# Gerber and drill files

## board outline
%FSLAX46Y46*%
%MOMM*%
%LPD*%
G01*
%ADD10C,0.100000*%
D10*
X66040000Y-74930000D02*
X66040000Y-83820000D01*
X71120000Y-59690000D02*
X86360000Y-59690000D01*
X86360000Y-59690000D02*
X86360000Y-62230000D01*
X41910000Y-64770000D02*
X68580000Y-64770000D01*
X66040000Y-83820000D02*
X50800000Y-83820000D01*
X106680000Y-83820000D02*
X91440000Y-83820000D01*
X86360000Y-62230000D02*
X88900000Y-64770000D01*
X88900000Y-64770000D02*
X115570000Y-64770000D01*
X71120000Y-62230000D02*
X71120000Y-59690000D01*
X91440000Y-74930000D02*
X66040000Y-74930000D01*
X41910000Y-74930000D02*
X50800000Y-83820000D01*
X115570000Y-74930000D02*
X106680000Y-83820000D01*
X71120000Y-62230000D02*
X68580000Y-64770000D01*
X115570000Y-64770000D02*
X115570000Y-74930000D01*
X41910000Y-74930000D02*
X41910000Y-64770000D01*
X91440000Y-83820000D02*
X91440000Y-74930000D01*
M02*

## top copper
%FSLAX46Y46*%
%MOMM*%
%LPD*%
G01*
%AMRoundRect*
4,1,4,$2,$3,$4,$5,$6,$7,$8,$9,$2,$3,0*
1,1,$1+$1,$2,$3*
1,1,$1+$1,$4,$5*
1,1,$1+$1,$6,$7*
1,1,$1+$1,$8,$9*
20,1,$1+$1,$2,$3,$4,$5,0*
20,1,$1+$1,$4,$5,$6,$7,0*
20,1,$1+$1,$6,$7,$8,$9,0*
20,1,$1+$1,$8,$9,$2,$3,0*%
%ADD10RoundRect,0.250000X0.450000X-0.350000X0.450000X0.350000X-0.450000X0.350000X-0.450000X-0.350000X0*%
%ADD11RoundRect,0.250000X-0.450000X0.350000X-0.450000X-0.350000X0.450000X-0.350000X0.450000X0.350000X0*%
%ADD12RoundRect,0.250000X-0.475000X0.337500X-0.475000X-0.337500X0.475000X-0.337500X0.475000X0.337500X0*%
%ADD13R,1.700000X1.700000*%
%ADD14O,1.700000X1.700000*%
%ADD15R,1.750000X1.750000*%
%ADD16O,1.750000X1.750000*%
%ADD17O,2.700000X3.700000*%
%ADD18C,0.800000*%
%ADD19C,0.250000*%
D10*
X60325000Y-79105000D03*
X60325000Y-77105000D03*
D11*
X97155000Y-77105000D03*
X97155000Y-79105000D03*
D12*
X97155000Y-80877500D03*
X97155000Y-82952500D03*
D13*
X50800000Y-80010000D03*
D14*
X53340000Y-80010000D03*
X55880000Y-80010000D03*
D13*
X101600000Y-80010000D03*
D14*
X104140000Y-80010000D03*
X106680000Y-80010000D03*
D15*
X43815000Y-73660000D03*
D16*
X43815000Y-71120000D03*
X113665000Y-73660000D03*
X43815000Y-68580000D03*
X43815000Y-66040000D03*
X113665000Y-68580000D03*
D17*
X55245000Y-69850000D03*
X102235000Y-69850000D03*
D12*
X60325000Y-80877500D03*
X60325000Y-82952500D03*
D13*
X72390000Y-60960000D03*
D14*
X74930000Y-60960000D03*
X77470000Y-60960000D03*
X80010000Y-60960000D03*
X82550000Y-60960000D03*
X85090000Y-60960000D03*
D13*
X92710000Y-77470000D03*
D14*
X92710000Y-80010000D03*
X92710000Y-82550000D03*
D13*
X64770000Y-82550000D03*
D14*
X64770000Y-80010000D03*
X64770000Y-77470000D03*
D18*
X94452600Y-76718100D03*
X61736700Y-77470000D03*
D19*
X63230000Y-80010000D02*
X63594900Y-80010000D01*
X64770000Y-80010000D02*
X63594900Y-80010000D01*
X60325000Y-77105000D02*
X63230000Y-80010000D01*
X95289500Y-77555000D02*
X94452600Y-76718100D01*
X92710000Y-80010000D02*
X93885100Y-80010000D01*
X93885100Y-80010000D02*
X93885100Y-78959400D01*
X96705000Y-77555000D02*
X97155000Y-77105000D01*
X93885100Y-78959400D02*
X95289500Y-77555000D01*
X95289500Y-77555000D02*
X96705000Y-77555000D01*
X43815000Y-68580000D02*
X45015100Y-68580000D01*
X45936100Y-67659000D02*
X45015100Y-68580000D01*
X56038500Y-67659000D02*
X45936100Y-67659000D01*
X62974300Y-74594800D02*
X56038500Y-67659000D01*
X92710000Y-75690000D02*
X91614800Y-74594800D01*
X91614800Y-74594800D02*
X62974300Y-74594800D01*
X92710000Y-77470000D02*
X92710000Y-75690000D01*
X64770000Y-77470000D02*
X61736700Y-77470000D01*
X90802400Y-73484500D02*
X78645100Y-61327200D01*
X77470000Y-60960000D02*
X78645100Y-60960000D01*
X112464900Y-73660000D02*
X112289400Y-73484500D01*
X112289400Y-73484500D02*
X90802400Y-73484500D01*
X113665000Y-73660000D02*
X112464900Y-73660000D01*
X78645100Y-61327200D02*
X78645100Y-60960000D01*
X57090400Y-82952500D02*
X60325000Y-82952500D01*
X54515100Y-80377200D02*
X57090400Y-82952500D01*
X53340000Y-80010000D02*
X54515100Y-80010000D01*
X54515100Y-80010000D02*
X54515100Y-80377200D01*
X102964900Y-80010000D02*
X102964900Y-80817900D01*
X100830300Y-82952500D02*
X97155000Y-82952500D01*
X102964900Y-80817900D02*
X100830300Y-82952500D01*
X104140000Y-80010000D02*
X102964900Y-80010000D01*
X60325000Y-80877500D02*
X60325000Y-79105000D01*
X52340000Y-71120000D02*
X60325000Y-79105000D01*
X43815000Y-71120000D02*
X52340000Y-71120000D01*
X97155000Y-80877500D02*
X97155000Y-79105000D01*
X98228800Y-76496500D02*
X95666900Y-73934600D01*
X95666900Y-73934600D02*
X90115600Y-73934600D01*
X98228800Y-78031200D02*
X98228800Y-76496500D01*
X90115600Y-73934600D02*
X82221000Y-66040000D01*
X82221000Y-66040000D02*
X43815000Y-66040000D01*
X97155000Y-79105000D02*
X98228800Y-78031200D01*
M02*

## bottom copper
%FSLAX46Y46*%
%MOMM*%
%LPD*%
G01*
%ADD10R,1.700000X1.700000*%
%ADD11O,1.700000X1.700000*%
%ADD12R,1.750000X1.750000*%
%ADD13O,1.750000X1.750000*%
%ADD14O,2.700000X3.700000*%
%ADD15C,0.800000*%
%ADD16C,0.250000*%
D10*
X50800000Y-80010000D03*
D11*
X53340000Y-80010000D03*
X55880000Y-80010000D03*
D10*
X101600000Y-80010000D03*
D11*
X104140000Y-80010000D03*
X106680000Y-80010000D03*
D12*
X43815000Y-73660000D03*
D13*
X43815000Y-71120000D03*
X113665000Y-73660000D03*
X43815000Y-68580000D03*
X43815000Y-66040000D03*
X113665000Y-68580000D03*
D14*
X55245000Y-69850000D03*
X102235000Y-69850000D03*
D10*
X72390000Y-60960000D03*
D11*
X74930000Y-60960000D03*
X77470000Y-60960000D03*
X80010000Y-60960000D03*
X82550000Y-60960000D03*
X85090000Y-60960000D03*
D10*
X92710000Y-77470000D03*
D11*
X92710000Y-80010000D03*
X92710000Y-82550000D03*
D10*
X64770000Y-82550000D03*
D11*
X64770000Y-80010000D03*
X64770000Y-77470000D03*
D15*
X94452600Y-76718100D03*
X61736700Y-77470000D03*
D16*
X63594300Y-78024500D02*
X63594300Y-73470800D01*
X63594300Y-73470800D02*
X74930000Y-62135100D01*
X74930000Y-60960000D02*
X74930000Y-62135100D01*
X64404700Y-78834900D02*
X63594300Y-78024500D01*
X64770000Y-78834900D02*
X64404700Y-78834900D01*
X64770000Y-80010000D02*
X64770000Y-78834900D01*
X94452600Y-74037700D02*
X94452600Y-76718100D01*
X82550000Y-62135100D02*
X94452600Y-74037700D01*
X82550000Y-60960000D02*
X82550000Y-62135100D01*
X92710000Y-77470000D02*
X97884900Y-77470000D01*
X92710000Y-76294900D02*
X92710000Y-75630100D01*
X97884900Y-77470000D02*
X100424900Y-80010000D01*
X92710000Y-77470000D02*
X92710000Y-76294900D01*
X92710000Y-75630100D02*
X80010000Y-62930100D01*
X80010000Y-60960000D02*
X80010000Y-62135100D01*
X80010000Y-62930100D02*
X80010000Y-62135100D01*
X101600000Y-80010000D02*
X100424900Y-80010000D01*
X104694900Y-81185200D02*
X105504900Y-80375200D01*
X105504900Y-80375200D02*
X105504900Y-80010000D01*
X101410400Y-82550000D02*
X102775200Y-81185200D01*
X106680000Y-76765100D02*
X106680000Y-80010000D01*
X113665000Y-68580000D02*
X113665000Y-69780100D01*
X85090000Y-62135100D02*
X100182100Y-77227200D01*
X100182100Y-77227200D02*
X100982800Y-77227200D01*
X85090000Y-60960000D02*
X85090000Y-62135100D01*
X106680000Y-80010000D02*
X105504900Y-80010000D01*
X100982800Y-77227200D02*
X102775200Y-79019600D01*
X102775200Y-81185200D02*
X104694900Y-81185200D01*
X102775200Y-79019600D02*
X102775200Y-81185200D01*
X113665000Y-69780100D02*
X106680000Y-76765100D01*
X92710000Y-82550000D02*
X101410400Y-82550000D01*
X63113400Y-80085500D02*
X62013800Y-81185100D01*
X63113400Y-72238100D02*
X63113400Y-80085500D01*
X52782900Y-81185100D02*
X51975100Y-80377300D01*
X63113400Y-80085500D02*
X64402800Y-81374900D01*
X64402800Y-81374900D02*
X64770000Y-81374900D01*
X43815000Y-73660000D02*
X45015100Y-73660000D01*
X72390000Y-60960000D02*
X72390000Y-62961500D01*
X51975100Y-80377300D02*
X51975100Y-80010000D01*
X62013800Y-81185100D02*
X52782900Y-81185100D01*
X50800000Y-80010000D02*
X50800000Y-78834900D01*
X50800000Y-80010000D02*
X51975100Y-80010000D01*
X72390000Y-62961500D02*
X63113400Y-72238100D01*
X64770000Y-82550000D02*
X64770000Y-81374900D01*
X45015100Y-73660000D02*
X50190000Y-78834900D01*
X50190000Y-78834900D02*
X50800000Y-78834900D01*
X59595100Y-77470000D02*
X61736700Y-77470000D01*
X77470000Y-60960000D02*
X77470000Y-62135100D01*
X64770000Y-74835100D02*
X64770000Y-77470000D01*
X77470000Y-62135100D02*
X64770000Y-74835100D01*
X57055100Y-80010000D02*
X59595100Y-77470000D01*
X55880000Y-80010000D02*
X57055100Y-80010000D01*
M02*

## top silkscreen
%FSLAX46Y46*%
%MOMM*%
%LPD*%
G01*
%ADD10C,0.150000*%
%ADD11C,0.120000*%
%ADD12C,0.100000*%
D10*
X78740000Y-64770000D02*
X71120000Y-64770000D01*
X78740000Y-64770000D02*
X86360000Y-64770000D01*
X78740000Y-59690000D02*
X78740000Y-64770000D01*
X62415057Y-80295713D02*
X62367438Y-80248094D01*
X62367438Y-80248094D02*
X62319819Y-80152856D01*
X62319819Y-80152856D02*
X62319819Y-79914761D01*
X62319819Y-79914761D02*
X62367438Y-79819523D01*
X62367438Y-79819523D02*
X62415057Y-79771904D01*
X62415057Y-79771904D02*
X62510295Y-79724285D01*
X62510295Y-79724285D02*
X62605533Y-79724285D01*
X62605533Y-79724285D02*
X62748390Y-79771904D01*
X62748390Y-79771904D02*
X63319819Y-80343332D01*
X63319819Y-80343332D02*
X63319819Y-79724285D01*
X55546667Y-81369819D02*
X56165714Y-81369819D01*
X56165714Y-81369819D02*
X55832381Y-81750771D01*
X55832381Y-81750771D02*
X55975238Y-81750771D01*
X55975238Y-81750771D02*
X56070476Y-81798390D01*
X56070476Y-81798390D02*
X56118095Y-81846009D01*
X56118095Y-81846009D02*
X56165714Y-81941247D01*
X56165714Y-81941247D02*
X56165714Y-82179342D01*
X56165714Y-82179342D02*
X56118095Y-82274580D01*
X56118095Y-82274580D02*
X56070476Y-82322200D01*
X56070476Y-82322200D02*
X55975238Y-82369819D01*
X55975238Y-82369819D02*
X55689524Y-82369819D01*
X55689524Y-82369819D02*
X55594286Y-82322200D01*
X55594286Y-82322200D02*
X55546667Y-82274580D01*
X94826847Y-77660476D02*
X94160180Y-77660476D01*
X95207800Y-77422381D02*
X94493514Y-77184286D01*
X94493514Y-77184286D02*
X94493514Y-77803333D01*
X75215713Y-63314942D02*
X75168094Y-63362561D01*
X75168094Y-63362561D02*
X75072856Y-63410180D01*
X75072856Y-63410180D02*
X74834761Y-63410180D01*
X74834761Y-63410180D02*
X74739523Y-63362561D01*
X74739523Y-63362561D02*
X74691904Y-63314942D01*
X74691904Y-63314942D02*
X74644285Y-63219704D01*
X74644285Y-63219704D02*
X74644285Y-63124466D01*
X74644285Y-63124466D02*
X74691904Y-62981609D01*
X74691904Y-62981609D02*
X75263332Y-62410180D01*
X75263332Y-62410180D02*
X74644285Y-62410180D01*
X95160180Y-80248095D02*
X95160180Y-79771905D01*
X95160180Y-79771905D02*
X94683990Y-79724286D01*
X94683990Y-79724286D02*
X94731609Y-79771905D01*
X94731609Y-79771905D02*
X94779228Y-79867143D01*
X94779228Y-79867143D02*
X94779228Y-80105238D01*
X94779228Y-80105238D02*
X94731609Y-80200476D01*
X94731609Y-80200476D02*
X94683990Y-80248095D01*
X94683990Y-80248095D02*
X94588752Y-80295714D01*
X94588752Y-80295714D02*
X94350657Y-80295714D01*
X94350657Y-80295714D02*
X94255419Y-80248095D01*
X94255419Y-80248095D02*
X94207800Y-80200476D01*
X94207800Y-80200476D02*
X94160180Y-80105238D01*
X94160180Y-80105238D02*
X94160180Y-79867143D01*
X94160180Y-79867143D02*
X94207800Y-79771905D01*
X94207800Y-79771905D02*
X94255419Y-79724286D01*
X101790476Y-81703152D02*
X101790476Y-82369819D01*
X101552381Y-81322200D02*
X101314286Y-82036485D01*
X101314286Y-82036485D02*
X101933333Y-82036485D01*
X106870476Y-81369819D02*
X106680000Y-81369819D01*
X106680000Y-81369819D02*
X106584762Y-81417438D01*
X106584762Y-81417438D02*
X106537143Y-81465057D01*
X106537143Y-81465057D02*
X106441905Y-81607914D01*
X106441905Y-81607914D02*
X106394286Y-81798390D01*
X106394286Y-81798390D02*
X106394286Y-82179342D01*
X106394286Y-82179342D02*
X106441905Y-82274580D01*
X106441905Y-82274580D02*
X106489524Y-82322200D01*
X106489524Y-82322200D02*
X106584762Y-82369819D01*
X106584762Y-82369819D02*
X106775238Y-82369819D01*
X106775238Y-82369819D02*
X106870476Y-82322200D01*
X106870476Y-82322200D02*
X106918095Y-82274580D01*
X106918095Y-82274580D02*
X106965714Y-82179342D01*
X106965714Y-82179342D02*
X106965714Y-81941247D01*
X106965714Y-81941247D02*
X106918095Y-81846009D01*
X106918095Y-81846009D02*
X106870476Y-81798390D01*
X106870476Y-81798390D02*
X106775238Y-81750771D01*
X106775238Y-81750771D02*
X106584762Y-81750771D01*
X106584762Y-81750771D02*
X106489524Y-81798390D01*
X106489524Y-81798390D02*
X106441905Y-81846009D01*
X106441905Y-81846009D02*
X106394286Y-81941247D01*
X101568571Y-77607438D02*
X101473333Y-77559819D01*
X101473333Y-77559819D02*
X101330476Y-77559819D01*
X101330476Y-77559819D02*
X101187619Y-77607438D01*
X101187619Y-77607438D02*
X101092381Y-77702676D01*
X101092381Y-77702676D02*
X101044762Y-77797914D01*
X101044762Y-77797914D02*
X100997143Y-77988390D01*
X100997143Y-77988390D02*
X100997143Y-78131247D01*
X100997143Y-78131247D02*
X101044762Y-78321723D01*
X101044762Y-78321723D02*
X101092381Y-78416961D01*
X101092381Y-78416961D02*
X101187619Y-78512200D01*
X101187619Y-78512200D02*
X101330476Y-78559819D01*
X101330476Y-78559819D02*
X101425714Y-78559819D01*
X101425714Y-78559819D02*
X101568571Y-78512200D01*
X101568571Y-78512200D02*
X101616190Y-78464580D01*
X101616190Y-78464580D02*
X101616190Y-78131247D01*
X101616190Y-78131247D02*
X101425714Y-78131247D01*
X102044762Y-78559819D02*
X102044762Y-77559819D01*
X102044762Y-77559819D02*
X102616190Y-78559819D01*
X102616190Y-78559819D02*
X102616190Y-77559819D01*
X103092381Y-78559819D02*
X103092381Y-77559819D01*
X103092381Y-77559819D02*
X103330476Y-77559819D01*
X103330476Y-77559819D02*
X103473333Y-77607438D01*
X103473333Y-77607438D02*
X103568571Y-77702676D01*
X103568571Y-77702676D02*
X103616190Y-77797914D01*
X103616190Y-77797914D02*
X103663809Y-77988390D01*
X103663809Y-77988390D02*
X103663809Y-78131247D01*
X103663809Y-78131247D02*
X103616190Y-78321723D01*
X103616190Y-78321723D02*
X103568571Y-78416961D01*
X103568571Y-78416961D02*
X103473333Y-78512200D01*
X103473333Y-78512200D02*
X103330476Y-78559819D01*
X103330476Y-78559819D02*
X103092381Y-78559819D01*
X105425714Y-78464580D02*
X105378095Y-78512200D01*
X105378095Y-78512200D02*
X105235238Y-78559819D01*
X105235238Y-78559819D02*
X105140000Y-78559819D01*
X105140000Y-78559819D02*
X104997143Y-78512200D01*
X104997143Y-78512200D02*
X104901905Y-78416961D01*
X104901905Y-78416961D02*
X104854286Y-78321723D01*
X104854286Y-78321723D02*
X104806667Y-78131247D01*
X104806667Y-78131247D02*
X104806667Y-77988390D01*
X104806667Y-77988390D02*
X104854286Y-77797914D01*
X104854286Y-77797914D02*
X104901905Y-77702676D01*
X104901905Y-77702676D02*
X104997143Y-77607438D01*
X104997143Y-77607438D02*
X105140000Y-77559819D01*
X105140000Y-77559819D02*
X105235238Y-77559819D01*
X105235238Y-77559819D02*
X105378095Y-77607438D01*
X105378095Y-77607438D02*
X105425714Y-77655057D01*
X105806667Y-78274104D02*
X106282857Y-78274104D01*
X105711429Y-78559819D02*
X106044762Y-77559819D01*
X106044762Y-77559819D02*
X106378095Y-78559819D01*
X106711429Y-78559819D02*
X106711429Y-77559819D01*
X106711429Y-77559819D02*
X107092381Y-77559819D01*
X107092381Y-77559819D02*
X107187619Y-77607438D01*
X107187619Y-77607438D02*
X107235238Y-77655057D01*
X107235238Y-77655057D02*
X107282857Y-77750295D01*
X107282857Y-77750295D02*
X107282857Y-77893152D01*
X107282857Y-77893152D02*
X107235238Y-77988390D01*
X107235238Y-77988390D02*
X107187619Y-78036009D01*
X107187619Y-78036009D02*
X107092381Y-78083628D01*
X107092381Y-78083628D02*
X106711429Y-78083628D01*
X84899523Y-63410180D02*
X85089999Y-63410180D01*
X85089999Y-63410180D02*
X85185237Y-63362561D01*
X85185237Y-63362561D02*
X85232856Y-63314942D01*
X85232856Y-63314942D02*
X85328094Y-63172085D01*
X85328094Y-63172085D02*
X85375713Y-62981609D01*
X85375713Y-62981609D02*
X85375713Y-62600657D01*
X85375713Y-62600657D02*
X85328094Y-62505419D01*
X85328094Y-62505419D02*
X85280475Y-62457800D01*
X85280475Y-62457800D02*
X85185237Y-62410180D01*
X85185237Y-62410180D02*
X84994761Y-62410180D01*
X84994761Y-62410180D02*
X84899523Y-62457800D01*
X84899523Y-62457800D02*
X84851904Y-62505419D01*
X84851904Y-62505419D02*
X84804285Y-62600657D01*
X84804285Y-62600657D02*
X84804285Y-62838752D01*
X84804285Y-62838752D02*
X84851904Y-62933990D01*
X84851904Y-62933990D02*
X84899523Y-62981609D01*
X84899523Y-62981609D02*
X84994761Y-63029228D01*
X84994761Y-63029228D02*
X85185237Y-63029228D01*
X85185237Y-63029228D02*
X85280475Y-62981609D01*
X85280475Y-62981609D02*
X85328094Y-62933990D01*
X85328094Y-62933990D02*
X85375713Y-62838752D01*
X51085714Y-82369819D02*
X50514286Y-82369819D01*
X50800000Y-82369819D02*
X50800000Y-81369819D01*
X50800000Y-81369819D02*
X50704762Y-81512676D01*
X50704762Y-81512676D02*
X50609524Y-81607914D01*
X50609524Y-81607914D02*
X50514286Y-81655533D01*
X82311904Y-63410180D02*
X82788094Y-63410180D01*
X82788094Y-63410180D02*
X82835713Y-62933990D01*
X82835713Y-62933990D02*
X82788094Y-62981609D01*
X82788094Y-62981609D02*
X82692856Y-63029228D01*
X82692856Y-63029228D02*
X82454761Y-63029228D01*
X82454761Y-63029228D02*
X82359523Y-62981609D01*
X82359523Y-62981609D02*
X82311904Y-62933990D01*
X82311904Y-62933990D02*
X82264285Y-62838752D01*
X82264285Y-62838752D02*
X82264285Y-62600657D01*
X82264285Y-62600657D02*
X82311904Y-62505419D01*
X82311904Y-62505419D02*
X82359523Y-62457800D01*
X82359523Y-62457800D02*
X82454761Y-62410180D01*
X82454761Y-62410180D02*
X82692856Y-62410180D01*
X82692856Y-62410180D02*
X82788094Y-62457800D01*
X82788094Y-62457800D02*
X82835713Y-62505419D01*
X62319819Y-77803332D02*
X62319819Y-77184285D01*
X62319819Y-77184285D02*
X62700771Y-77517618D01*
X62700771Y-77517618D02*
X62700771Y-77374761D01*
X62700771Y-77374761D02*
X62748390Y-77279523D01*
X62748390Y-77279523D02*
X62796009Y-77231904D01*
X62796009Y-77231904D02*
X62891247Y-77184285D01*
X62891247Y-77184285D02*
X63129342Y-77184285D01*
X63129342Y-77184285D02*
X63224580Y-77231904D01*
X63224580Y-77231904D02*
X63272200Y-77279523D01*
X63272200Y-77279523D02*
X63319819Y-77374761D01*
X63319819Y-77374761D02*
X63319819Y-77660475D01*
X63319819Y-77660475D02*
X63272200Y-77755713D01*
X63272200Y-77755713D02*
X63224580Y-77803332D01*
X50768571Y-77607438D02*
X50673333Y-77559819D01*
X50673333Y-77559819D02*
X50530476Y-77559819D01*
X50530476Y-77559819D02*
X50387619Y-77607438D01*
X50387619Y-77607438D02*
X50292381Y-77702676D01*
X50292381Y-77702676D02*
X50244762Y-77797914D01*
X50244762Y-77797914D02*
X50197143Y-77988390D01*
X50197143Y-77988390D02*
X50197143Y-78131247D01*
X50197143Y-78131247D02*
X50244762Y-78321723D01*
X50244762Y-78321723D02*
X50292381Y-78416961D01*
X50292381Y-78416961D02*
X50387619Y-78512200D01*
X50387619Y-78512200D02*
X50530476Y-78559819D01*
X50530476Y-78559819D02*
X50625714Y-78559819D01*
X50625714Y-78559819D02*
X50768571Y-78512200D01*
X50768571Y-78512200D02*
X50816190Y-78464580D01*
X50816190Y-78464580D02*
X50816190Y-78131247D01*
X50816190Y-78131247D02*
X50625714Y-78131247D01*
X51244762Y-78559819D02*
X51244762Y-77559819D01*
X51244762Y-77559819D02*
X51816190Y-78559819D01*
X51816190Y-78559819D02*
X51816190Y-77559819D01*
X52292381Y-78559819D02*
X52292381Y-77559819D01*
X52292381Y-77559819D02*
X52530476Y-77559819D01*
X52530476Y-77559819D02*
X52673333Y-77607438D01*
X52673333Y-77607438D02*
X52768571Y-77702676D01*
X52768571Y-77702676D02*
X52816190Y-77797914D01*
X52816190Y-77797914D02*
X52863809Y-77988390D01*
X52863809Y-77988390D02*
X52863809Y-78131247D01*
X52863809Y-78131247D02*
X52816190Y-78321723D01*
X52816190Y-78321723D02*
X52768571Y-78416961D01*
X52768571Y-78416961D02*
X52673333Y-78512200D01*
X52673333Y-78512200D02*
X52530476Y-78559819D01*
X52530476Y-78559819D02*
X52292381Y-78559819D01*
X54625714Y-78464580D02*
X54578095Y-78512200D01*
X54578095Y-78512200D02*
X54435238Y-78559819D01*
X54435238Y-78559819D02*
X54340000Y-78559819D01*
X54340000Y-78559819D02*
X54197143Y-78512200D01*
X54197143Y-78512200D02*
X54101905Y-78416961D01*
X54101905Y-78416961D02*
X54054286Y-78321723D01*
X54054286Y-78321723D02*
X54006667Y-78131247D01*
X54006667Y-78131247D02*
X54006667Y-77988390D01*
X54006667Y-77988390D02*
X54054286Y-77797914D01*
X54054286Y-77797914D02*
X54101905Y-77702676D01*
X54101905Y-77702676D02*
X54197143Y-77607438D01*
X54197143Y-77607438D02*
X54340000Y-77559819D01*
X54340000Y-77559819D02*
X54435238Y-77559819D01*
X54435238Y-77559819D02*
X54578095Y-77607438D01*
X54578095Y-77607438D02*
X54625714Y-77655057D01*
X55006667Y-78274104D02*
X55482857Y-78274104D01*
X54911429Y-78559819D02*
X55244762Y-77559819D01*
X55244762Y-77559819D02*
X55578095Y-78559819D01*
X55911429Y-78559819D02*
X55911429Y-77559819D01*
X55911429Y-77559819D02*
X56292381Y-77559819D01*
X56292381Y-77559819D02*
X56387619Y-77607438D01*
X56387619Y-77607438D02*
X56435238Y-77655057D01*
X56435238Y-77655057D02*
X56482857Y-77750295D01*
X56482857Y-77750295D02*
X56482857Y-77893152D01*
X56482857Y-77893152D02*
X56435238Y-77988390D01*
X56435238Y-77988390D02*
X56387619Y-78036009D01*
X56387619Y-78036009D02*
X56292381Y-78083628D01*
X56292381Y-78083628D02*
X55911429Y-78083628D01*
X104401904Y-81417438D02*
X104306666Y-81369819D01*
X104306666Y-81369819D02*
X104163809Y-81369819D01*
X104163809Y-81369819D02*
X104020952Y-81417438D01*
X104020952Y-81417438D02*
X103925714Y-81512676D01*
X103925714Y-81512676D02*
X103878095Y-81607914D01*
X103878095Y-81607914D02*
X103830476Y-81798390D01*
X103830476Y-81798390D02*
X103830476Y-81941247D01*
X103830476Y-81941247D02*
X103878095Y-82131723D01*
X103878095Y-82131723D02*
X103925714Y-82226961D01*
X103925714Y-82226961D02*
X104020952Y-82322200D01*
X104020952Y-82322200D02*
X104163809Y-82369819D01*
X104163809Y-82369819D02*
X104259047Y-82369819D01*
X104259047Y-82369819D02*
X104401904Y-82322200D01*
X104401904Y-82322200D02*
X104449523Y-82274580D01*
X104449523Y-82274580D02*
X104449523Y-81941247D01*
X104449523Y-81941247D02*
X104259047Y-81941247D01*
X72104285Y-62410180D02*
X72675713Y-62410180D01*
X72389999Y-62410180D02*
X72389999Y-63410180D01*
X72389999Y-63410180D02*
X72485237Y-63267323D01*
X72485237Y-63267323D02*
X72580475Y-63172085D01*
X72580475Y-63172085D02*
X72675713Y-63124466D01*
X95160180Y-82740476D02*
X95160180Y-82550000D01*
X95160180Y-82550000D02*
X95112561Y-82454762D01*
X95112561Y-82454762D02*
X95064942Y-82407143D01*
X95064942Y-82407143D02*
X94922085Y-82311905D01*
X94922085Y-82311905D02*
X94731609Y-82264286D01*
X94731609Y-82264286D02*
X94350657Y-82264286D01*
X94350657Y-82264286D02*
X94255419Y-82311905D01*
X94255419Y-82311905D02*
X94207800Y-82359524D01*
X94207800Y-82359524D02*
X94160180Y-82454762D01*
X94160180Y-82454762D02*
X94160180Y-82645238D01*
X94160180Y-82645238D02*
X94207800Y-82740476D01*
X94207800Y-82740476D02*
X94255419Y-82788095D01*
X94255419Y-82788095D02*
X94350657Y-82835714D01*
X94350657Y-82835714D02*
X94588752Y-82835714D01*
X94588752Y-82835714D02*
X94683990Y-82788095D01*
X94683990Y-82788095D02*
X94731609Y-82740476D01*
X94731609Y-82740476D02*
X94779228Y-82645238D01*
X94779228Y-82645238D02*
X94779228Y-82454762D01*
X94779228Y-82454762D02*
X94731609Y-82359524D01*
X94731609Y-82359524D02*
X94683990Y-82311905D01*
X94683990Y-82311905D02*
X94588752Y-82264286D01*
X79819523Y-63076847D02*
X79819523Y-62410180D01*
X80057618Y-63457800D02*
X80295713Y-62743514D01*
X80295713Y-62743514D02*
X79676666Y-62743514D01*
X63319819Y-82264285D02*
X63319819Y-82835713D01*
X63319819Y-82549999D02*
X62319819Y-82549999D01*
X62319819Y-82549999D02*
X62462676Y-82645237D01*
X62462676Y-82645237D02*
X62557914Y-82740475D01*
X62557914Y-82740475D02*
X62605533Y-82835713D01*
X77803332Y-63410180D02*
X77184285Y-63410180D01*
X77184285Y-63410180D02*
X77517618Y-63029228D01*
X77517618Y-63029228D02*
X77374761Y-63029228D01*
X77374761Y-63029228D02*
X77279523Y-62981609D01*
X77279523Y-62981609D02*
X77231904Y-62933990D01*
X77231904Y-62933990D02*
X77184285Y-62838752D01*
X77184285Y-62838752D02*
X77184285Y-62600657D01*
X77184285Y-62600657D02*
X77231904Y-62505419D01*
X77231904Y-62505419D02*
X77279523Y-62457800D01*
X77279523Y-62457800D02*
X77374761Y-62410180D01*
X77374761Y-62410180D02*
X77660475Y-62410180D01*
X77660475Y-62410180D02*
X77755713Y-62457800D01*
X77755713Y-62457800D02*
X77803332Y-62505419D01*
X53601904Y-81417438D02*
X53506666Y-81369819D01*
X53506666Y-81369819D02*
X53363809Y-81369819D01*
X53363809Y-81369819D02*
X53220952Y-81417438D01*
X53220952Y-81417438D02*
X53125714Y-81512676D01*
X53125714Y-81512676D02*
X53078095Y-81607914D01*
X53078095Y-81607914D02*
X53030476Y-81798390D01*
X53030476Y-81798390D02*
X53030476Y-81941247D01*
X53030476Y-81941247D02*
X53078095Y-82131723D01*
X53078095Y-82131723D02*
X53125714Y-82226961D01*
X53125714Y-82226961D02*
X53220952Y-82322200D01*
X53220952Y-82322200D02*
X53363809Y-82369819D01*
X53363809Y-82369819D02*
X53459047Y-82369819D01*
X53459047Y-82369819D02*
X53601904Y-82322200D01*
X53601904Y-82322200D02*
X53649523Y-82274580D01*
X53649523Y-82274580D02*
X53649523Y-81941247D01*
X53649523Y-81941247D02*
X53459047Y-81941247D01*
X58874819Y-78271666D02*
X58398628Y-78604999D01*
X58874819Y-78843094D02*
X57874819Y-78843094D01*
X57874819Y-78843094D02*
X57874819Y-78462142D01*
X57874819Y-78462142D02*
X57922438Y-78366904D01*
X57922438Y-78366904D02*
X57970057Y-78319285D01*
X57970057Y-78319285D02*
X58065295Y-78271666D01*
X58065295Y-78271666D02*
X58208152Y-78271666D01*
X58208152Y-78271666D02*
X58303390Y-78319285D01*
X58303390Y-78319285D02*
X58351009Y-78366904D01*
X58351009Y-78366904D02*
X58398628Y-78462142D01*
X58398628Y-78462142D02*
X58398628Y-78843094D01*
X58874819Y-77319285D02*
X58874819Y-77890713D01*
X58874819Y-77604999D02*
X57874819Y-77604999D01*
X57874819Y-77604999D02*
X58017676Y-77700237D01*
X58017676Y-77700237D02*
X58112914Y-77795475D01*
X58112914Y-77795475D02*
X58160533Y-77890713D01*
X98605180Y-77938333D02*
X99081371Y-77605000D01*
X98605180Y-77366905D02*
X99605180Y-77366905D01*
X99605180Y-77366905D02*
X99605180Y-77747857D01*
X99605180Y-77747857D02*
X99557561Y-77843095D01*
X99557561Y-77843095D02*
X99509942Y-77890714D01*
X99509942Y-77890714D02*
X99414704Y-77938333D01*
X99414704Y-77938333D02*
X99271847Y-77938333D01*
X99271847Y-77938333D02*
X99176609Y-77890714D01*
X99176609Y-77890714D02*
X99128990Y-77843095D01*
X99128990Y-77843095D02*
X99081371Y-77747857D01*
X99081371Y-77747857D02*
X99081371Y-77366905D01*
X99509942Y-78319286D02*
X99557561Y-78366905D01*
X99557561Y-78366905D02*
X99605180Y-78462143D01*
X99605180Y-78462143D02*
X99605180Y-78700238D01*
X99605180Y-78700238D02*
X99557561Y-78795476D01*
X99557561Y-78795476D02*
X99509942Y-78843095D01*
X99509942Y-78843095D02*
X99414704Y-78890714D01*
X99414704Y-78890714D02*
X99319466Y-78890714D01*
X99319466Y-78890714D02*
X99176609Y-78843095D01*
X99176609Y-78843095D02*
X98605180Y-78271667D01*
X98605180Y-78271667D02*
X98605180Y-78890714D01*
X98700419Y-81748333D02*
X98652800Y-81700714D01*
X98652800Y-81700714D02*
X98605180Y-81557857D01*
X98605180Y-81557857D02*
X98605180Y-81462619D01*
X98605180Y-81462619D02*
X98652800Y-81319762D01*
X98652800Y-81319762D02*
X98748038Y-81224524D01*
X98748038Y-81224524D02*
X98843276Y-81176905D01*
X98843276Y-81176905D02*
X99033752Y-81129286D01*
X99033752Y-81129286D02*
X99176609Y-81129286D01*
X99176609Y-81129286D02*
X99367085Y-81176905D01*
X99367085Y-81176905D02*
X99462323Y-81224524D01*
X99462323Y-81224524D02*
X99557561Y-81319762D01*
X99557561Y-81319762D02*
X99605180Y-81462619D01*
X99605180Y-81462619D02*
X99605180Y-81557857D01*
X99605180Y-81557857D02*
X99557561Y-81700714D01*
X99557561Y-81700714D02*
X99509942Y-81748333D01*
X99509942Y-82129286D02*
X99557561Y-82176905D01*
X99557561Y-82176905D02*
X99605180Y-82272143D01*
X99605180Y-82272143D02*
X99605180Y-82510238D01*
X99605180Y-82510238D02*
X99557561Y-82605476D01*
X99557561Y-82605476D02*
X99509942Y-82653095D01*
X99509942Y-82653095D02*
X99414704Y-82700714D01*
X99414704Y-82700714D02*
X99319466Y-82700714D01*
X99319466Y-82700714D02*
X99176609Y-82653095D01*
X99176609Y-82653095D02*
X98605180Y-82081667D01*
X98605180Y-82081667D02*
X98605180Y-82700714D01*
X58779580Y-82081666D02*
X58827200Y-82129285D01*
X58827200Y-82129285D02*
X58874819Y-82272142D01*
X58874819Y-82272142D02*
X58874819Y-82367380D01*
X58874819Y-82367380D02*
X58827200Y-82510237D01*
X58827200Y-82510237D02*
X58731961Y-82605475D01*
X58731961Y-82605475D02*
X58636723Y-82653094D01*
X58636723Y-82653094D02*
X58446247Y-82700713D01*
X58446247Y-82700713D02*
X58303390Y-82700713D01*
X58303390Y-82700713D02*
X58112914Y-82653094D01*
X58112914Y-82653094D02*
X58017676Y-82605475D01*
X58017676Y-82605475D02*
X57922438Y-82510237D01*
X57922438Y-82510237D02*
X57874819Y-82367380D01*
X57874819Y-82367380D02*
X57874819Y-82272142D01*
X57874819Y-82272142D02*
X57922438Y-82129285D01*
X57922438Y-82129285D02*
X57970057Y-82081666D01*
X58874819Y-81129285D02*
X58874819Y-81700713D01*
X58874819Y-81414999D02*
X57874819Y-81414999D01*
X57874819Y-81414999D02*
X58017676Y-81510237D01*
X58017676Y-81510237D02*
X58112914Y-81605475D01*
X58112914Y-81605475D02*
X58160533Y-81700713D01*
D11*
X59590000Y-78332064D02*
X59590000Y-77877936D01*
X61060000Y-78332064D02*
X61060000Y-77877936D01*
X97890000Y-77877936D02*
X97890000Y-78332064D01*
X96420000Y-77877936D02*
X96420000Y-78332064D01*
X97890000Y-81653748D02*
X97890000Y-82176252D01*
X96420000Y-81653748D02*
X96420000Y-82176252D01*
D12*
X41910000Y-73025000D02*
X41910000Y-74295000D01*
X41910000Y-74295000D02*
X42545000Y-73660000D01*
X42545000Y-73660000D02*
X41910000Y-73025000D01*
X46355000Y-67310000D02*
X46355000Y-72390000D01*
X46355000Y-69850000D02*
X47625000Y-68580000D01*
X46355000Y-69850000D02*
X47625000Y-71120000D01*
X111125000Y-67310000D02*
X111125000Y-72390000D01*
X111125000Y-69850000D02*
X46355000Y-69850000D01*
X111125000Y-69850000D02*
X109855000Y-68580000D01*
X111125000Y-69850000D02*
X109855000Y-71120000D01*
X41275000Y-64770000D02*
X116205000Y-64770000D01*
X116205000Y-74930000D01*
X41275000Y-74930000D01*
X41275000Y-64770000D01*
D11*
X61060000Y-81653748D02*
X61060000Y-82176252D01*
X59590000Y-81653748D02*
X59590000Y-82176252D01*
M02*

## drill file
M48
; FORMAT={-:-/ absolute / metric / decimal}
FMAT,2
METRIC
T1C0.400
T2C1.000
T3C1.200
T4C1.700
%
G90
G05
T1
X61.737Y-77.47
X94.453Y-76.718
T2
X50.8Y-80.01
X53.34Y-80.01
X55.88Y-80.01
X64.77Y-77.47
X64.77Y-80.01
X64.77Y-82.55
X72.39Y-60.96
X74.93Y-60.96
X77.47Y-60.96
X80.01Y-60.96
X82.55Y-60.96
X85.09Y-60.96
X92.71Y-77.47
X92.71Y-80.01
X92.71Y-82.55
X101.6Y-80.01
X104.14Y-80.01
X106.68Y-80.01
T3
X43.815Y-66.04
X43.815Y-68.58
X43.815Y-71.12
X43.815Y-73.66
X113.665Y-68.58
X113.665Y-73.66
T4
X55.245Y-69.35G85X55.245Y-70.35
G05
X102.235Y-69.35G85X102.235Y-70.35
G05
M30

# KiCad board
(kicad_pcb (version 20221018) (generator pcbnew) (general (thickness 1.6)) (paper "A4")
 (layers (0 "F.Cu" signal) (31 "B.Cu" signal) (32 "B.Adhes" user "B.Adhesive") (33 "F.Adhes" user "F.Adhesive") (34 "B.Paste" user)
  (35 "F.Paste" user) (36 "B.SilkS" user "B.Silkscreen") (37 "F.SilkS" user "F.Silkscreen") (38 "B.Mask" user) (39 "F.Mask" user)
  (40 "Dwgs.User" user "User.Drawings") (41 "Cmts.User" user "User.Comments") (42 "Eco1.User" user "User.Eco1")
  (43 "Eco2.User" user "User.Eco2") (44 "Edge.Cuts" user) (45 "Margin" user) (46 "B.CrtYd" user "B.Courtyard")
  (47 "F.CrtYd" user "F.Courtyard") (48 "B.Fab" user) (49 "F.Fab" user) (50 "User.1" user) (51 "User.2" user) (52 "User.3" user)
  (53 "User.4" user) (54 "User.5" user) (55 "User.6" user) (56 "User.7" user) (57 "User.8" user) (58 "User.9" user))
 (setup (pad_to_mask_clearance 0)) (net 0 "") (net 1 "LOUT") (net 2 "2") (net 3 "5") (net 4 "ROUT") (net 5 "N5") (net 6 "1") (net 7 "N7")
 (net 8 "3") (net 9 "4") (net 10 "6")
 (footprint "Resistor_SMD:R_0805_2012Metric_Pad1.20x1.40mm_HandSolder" (layer "F.Cu") (at 60.325 78.105 90)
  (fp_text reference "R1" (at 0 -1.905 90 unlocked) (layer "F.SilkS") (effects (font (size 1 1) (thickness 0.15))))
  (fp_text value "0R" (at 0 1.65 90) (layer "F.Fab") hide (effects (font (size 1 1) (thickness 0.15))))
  (fp_line (start -0.227064 -0.735) (end 0.227064 -0.735) (stroke (width 0.12) (type solid)) (layer "F.SilkS"))
  (fp_line (start -0.227064 0.735) (end 0.227064 0.735) (stroke (width 0.12) (type solid)) (layer "F.SilkS"))
  (pad "1" smd roundrect (at -1 0 90) (size 1.2 1.4) (layers "F.Cu" "F.Paste" "F.Mask") (roundrect_rratio 0.208333) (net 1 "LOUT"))
  (pad "2" smd roundrect (at 1 0 90) (size 1.2 1.4) (layers "F.Cu" "F.Paste" "F.Mask") (roundrect_rratio 0.208333) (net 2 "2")))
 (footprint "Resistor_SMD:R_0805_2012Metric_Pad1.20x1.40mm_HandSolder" (layer "F.Cu") (at 97.155 78.105 -90)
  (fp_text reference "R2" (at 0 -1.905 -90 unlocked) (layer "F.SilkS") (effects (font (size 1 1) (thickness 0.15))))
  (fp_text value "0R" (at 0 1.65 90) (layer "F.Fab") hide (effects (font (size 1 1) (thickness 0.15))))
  (fp_line (start -0.227064 -0.735) (end 0.227064 -0.735) (stroke (width 0.12) (type solid)) (layer "F.SilkS"))
  (fp_line (start -0.227064 0.735) (end 0.227064 0.735) (stroke (width 0.12) (type solid)) (layer "F.SilkS"))
  (pad "1" smd roundrect (at -1 0 270) (size 1.2 1.4) (layers "F.Cu" "F.Paste" "F.Mask") (roundrect_rratio 0.208333) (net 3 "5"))
  (pad "2" smd roundrect (at 1 0 270) (size 1.2 1.4) (layers "F.Cu" "F.Paste" "F.Mask") (roundrect_rratio 0.208333) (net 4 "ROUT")))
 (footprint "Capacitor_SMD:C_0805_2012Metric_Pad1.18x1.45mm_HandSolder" (layer "F.Cu") (at 97.155 81.915 -90)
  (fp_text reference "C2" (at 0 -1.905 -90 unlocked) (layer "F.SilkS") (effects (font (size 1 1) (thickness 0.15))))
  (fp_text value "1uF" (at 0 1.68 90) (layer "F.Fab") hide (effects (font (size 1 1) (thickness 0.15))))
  (fp_line (start -0.261252 -0.735) (end 0.261252 -0.735) (stroke (width 0.12) (type solid)) (layer "F.SilkS"))
  (fp_line (start -0.261252 0.735) (end 0.261252 0.735) (stroke (width 0.12) (type solid)) (layer "F.SilkS"))
  (pad "1" smd roundrect (at -1.0375 0 270) (size 1.175 1.45) (layers "F.Cu" "F.Paste" "F.Mask") (roundrect_rratio 0.212766) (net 4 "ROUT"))
  (pad "2" smd roundrect (at 1.0375 0 270) (size 1.175 1.45) (layers "F.Cu" "F.Paste" "F.Mask") (roundrect_rratio 0.212766) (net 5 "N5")))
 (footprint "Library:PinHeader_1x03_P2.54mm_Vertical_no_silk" (layer "F.Cu") (at 50.8 80.01 90)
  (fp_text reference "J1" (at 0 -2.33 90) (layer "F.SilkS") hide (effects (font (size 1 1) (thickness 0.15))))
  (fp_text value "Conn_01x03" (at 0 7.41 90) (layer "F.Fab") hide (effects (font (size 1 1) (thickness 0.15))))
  (pad "1" thru_hole rect (at 0 0 90) (size 1.7 1.7) (drill 1) (layers "*.Cu" "*.Mask") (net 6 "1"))
  (pad "2" thru_hole oval (at 0 2.54 90) (size 1.7 1.7) (drill 1) (layers "*.Cu" "*.Mask") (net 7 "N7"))
  (pad "3" thru_hole oval (at 0 5.08 90) (size 1.7 1.7) (drill 1) (layers "*.Cu" "*.Mask") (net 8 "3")))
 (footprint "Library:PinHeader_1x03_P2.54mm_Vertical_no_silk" (layer "F.Cu") (at 101.6 80.01 90)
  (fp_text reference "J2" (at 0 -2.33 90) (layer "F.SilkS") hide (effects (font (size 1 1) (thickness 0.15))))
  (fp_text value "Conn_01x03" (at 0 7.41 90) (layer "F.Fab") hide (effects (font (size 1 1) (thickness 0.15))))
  (pad "1" thru_hole rect (at 0 0 90) (size 1.7 1.7) (drill 1) (layers "*.Cu" "*.Mask") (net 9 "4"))
  (pad "2" thru_hole oval (at 0 2.54 90) (size 1.7 1.7) (drill 1) (layers "*.Cu" "*.Mask") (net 5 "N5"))
  (pad "3" thru_hole oval (at 0 5.08 90) (size 1.7 1.7) (drill 1) (layers "*.Cu" "*.Mask") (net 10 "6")))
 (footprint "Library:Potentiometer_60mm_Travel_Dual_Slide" (layer "F.Cu") (at 78.74 69.85)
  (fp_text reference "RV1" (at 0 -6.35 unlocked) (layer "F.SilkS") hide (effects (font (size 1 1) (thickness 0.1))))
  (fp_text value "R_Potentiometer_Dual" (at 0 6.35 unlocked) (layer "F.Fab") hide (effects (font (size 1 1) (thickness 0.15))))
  (fp_line (start -36.83 3.175) (end -36.83 4.445) (stroke (width 0.1) (type default)) (layer "F.SilkS"))
  (fp_line (start -36.83 4.445) (end -36.195 3.81) (stroke (width 0.1) (type default)) (layer "F.SilkS"))
  (fp_line (start -36.195 3.81) (end -36.83 3.175) (stroke (width 0.1) (type default)) (layer "F.SilkS"))
  (fp_line (start -32.385 -2.54) (end -32.385 2.54) (stroke (width 0.1) (type default)) (layer "F.SilkS"))
  (fp_line (start -32.385 0) (end -31.115 -1.27) (stroke (width 0.1) (type default)) (layer "F.SilkS"))
  (fp_line (start -32.385 0) (end -31.115 1.27) (stroke (width 0.1) (type default)) (layer "F.SilkS"))
  (fp_line (start 32.385 -2.54) (end 32.385 2.54) (stroke (width 0.1) (type default)) (layer "F.SilkS"))
  (fp_line (start 32.385 0) (end -32.385 0) (stroke (width 0.1) (type default)) (layer "F.SilkS"))
  (fp_line (start 32.385 0) (end 31.115 -1.27) (stroke (width 0.1) (type default)) (layer "F.SilkS"))
  (fp_line (start 32.385 0) (end 31.115 1.27) (stroke (width 0.1) (type default)) (layer "F.SilkS"))
  (fp_rect (start -37.465 -5.08) (end 37.465 5.08) (stroke (width 0.1) (type default)) (fill none) (layer "F.SilkS"))
  (pad "1" thru_hole rect (at -34.925 3.81) (size 1.75 1.75) (drill 1.2) (layers "*.Cu" "*.Mask") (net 6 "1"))
  (pad "2" thru_hole oval (at -34.925 1.27) (size 1.75 1.75) (drill 1.2) (layers "*.Cu" "*.Mask") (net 1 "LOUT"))
  (pad "3" thru_hole oval (at 34.925 3.81) (size 1.75 1.75) (drill 1.2) (layers "*.Cu" "*.Mask") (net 8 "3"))
  (pad "4" thru_hole oval (at -34.925 -1.27) (size 1.75 1.75) (drill 1.2) (layers "*.Cu" "*.Mask") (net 9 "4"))
  (pad "5" thru_hole oval (at -34.925 -3.81) (size 1.75 1.75) (drill 1.2) (layers "*.Cu" "*.Mask") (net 4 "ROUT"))
  (pad "6" thru_hole oval (at 34.925 -1.27) (size 1.75 1.75) (drill 1.2) (layers "*.Cu" "*.Mask") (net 10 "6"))
  (pad "MP" thru_hole oval (at -23.495 0) (size 2.7 3.7) (drill oval 1.7 2.7) (layers "*.Cu" "*.Mask"))
  (pad "MP" thru_hole oval (at 23.495 0) (size 2.7 3.7) (drill oval 1.7 2.7) (layers "*.Cu" "*.Mask")))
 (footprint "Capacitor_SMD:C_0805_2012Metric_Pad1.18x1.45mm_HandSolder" (layer "F.Cu") (at 60.325 81.915 -90)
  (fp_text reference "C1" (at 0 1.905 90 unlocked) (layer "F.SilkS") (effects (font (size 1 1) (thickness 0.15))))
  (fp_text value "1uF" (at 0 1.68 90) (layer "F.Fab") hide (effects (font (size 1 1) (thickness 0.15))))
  (fp_line (start -0.261252 -0.735) (end 0.261252 -0.735) (stroke (width 0.12) (type solid)) (layer "F.SilkS"))
  (fp_line (start -0.261252 0.735) (end 0.261252 0.735) (stroke (width 0.12) (type solid)) (layer "F.SilkS"))
  (pad "1" smd roundrect (at -1.0375 0 270) (size 1.175 1.45) (layers "F.Cu" "F.Paste" "F.Mask") (roundrect_rratio 0.212766) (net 1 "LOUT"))
  (pad "2" smd roundrect (at 1.0375 0 270) (size 1.175 1.45) (layers "F.Cu" "F.Paste" "F.Mask") (roundrect_rratio 0.212766) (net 7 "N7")))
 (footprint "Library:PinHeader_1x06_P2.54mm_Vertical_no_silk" (layer "B.Cu") (at 72.39 60.96 -90)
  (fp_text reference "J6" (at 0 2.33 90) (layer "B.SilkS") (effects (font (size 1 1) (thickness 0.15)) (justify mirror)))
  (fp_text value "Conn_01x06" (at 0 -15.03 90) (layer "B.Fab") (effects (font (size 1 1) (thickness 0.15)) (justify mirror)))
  (pad "1" thru_hole rect (at 0 0 270) (size 1.7 1.7) (drill 1) (layers "*.Cu" "*.Mask") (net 6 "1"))
  (pad "2" thru_hole oval (at 0 -2.54 270) (size 1.7 1.7) (drill 1) (layers "*.Cu" "*.Mask") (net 2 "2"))
  (pad "3" thru_hole oval (at 0 -5.08 270) (size 1.7 1.7) (drill 1) (layers "*.Cu" "*.Mask") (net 8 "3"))
  (pad "4" thru_hole oval (at 0 -7.62 270) (size 1.7 1.7) (drill 1) (layers "*.Cu" "*.Mask") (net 9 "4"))
  (pad "5" thru_hole oval (at 0 -10.16 270) (size 1.7 1.7) (drill 1) (layers "*.Cu" "*.Mask") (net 3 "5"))
  (pad "6" thru_hole oval (at 0 -12.7 270) (size 1.7 1.7) (drill 1) (layers "*.Cu" "*.Mask") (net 10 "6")))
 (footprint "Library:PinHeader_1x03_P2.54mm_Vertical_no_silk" (layer "B.Cu") (at 92.71 77.47 180)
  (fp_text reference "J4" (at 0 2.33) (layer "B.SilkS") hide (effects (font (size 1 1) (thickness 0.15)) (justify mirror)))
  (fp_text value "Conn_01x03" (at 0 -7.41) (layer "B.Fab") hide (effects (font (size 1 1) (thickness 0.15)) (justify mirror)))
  (pad "1" thru_hole rect (at 0 0 180) (size 1.7 1.7) (drill 1) (layers "*.Cu" "*.Mask") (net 9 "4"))
  (pad "2" thru_hole oval (at 0 -2.54 180) (size 1.7 1.7) (drill 1) (layers "*.Cu" "*.Mask") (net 3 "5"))
  (pad "3" thru_hole oval (at 0 -5.08 180) (size 1.7 1.7) (drill 1) (layers "*.Cu" "*.Mask") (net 10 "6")))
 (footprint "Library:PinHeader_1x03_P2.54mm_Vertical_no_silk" (layer "B.Cu") (at 64.77 82.55)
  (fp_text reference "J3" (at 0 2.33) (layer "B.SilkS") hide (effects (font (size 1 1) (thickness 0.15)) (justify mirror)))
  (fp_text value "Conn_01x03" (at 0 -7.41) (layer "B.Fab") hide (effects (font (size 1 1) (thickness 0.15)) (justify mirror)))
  (pad "1" thru_hole rect (at 0 0) (size 1.7 1.7) (drill 1) (layers "*.Cu" "*.Mask") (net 6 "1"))
  (pad "2" thru_hole oval (at 0 -2.54) (size 1.7 1.7) (drill 1) (layers "*.Cu" "*.Mask") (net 2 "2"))
  (pad "3" thru_hole oval (at 0 -5.08) (size 1.7 1.7) (drill 1) (layers "*.Cu" "*.Mask") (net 8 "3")))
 (gr_line (start 78.74 64.77) (end 71.12 64.77) (stroke (width 0.15) (type default)) (layer "F.SilkS"))
 (gr_line (start 78.74 64.77) (end 86.36 64.77) (stroke (width 0.15) (type default)) (layer "F.SilkS"))
 (gr_line (start 78.74 59.69) (end 78.74 64.77) (stroke (width 0.15) (type default)) (layer "F.SilkS"))
 (gr_line (start 66.04 74.93) (end 66.04 83.82) (stroke (width 0.1) (type default)) (layer "Edge.Cuts"))
 (gr_line (start 71.12 59.69) (end 86.36 59.69) (stroke (width 0.1) (type default)) (layer "Edge.Cuts"))
 (gr_line (start 86.36 59.69) (end 86.36 62.23) (stroke (width 0.1) (type default)) (layer "Edge.Cuts"))
 (gr_line (start 41.91 64.77) (end 68.58 64.77) (stroke (width 0.1) (type default)) (layer "Edge.Cuts"))
 (gr_line (start 66.04 83.82) (end 50.8 83.82) (stroke (width 0.1) (type default)) (layer "Edge.Cuts"))
 (gr_line (start 106.68 83.82) (end 91.44 83.82) (stroke (width 0.1) (type default)) (layer "Edge.Cuts"))
 (gr_line (start 86.36 62.23) (end 88.9 64.77) (stroke (width 0.1) (type default)) (layer "Edge.Cuts"))
 (gr_line (start 88.9 64.77) (end 115.57 64.77) (stroke (width 0.1) (type default)) (layer "Edge.Cuts"))
 (gr_line (start 71.12 62.23) (end 71.12 59.69) (stroke (width 0.1) (type default)) (layer "Edge.Cuts"))
 (gr_line (start 91.44 74.93) (end 66.04 74.93) (stroke (width 0.1) (type default)) (layer "Edge.Cuts"))
 (gr_line (start 41.91 74.93) (end 50.8 83.82) (stroke (width 0.1) (type default)) (layer "Edge.Cuts"))
 (gr_line (start 115.57 74.93) (end 106.68 83.82) (stroke (width 0.1) (type default)) (layer "Edge.Cuts"))
 (gr_line (start 71.12 62.23) (end 68.58 64.77) (stroke (width 0.1) (type default)) (layer "Edge.Cuts"))
 (gr_line (start 115.57 64.77) (end 115.57 74.93) (stroke (width 0.1) (type default)) (layer "Edge.Cuts"))
 (gr_line (start 41.91 74.93) (end 41.91 64.77) (stroke (width 0.1) (type default)) (layer "Edge.Cuts"))
 (gr_line (start 91.44 83.82) (end 91.44 74.93) (stroke (width 0.1) (type default)) (layer "Edge.Cuts"))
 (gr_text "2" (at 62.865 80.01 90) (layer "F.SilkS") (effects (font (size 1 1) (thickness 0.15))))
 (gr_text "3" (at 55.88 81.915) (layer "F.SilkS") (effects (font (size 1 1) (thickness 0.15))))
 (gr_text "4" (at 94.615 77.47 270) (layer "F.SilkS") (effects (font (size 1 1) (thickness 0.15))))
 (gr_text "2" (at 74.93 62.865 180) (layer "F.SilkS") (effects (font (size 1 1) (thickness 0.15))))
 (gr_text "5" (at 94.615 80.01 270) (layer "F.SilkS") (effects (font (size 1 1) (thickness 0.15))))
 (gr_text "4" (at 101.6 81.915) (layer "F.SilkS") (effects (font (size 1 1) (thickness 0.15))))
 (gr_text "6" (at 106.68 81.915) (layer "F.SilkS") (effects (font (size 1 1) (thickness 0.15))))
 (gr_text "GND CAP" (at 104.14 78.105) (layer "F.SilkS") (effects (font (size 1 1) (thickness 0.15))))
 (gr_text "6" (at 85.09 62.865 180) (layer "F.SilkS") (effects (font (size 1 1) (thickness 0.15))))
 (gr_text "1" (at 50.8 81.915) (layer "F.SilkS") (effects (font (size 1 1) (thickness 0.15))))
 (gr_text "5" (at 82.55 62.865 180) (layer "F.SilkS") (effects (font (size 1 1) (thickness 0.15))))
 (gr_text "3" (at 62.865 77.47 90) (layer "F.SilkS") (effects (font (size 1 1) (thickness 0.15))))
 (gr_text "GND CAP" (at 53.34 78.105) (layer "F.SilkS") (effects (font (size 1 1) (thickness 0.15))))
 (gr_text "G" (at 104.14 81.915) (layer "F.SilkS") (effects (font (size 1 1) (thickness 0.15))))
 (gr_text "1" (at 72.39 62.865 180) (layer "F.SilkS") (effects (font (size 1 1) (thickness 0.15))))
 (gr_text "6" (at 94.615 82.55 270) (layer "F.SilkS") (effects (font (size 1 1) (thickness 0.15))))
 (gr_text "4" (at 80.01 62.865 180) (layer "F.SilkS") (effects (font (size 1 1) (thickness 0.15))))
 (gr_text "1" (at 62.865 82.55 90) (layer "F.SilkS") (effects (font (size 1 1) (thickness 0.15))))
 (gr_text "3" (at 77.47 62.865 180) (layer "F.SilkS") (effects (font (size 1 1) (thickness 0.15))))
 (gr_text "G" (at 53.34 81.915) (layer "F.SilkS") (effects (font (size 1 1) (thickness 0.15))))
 (segment (start 63.23 80.01) (end 63.5949 80.01) (width 0.25) (layer "F.Cu") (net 2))
 (segment (start 64.77 80.01) (end 63.5949 80.01) (width 0.25) (layer "F.Cu") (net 2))
 (segment (start 60.325 77.105) (end 63.23 80.01) (width 0.25) (layer "F.Cu") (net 2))
 (segment (start 63.5943 78.0245) (end 63.5943 73.4708) (width 0.25) (layer "B.Cu") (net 2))
 (segment (start 63.5943 73.4708) (end 74.93 62.1351) (width 0.25) (layer "B.Cu") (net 2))
 (segment (start 74.93 60.96) (end 74.93 62.1351) (width 0.25) (layer "B.Cu") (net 2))
 (segment (start 64.4047 78.8349) (end 63.5943 78.0245) (width 0.25) (layer "B.Cu") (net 2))
 (segment (start 64.77 78.8349) (end 64.4047 78.8349) (width 0.25) (layer "B.Cu") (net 2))
 (segment (start 64.77 80.01) (end 64.77 78.8349) (width 0.25) (layer "B.Cu") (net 2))
 (segment (start 95.2895 77.555) (end 94.4526 76.7181) (width 0.25) (layer "F.Cu") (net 3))
 (segment (start 92.71 80.01) (end 93.8851 80.01) (width 0.25) (layer "F.Cu") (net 3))
 (segment (start 93.8851 80.01) (end 93.8851 78.9594) (width 0.25) (layer "F.Cu") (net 3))
 (segment (start 96.705 77.555) (end 97.155 77.105) (width 0.25) (layer "F.Cu") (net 3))
 (segment (start 93.8851 78.9594) (end 95.2895 77.555) (width 0.25) (layer "F.Cu") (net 3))
 (segment (start 95.2895 77.555) (end 96.705 77.555) (width 0.25) (layer "F.Cu") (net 3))
 (via (at 94.4526 76.7181) (size 0.8) (drill 0.4) (layers "F.Cu" "B.Cu") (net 3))
 (segment (start 94.4526 74.0377) (end 94.4526 76.7181) (width 0.25) (layer "B.Cu") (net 3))
 (segment (start 82.55 62.1351) (end 94.4526 74.0377) (width 0.25) (layer "B.Cu") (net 3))
 (segment (start 82.55 60.96) (end 82.55 62.1351) (width 0.25) (layer "B.Cu") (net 3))
 (segment (start 43.815 68.58) (end 45.0151 68.58) (width 0.25) (layer "F.Cu") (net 9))
 (segment (start 45.9361 67.659) (end 45.0151 68.58) (width 0.25) (layer "F.Cu") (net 9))
 (segment (start 56.0385 67.659) (end 45.9361 67.659) (width 0.25) (layer "F.Cu") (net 9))
 (segment (start 62.9743 74.5948) (end 56.0385 67.659) (width 0.25) (layer "F.Cu") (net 9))
 (segment (start 92.71 75.69) (end 91.6148 74.5948) (width 0.25) (layer "F.Cu") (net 9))
 (segment (start 91.6148 74.5948) (end 62.9743 74.5948) (width 0.25) (layer "F.Cu") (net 9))
 (segment (start 92.71 77.47) (end 92.71 75.69) (width 0.25) (layer "F.Cu") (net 9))
 (segment (start 92.71 77.47) (end 97.8849 77.47) (width 0.25) (layer "B.Cu") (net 9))
 (segment (start 92.71 76.2949) (end 92.71 75.6301) (width 0.25) (layer "B.Cu") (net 9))
 (segment (start 97.8849 77.47) (end 100.4249 80.01) (width 0.25) (layer "B.Cu") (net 9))
 (segment (start 92.71 77.47) (end 92.71 76.2949) (width 0.25) (layer "B.Cu") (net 9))
 (segment (start 92.71 75.6301) (end 80.01 62.9301) (width 0.25) (layer "B.Cu") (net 9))
 (segment (start 80.01 60.96) (end 80.01 62.1351) (width 0.25) (layer "B.Cu") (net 9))
 (segment (start 80.01 62.9301) (end 80.01 62.1351) (width 0.25) (layer "B.Cu") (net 9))
 (segment (start 101.6 80.01) (end 100.4249 80.01) (width 0.25) (layer "B.Cu") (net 9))
 (segment (start 104.6949 81.1852) (end 105.5049 80.3752) (width 0.25) (layer "B.Cu") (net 10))
 (segment (start 105.5049 80.3752) (end 105.5049 80.01) (width 0.25) (layer "B.Cu") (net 10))
 (segment (start 101.4104 82.55) (end 102.7752 81.1852) (width 0.25) (layer "B.Cu") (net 10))
 (segment (start 106.68 76.7651) (end 106.68 80.01) (width 0.25) (layer "B.Cu") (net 10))
 (segment (start 113.665 68.58) (end 113.665 69.7801) (width 0.25) (layer "B.Cu") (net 10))
 (segment (start 85.09 62.1351) (end 100.1821 77.2272) (width 0.25) (layer "B.Cu") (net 10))
 (segment (start 100.1821 77.2272) (end 100.9828 77.2272) (width 0.25) (layer "B.Cu") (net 10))
 (segment (start 85.09 60.96) (end 85.09 62.1351) (width 0.25) (layer "B.Cu") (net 10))
 (segment (start 106.68 80.01) (end 105.5049 80.01) (width 0.25) (layer "B.Cu") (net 10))
 (segment (start 100.9828 77.2272) (end 102.7752 79.0196) (width 0.25) (layer "B.Cu") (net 10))
 (segment (start 102.7752 81.1852) (end 104.6949 81.1852) (width 0.25) (layer "B.Cu") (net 10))
 (segment (start 102.7752 79.0196) (end 102.7752 81.1852) (width 0.25) (layer "B.Cu") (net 10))
 (segment (start 113.665 69.7801) (end 106.68 76.7651) (width 0.25) (layer "B.Cu") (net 10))
 (segment (start 92.71 82.55) (end 101.4104 82.55) (width 0.25) (layer "B.Cu") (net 10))
 (segment (start 63.1134 80.0855) (end 62.0138 81.1851) (width 0.25) (layer "B.Cu") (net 6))
 (segment (start 63.1134 72.2381) (end 63.1134 80.0855) (width 0.25) (layer "B.Cu") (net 6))
 (segment (start 52.7829 81.1851) (end 51.9751 80.3773) (width 0.25) (layer "B.Cu") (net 6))
 (segment (start 63.1134 80.0855) (end 64.4028 81.3749) (width 0.25) (layer "B.Cu") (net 6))
 (segment (start 64.4028 81.3749) (end 64.77 81.3749) (width 0.25) (layer "B.Cu") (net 6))
 (segment (start 43.815 73.66) (end 45.0151 73.66) (width 0.25) (layer "B.Cu") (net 6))
 (segment (start 72.39 60.96) (end 72.39 62.9615) (width 0.25) (layer "B.Cu") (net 6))
 (segment (start 51.9751 80.3773) (end 51.9751 80.01) (width 0.25) (layer "B.Cu") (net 6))
 (segment (start 62.0138 81.1851) (end 52.7829 81.1851) (width 0.25) (layer "B.Cu") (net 6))
 (segment (start 50.8 80.01) (end 50.8 78.8349) (width 0.25) (layer "B.Cu") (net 6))
 (segment (start 50.8 80.01) (end 51.9751 80.01) (width 0.25) (layer "B.Cu") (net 6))
 (segment (start 72.39 62.9615) (end 63.1134 72.2381) (width 0.25) (layer "B.Cu") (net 6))
 (segment (start 64.77 82.55) (end 64.77 81.3749) (width 0.25) (layer "B.Cu") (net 6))
 (segment (start 45.0151 73.66) (end 50.19 78.8349) (width 0.25) (layer "B.Cu") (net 6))
 (segment (start 50.19 78.8349) (end 50.8 78.8349) (width 0.25) (layer "B.Cu") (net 6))
 (segment (start 64.77 77.47) (end 61.7367 77.47) (width 0.25) (layer "F.Cu") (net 8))
 (segment (start 90.8024 73.4845) (end 78.6451 61.3272) (width 0.25) (layer "F.Cu") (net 8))
 (segment (start 77.47 60.96) (end 78.6451 60.96) (width 0.25) (layer "F.Cu") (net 8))
 (segment (start 112.4649 73.66) (end 112.2894 73.4845) (width 0.25) (layer "F.Cu") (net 8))
 (segment (start 112.2894 73.4845) (end 90.8024 73.4845) (width 0.25) (layer "F.Cu") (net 8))
 (segment (start 113.665 73.66) (end 112.4649 73.66) (width 0.25) (layer "F.Cu") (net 8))
 (segment (start 78.6451 61.3272) (end 78.6451 60.96) (width 0.25) (layer "F.Cu") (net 8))
 (via (at 61.7367 77.47) (size 0.8) (drill 0.4) (layers "F.Cu" "B.Cu") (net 8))
 (segment (start 59.5951 77.47) (end 61.7367 77.47) (width 0.25) (layer "B.Cu") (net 8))
 (segment (start 77.47 60.96) (end 77.47 62.1351) (width 0.25) (layer "B.Cu") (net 8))
 (segment (start 64.77 74.8351) (end 64.77 77.47) (width 0.25) (layer "B.Cu") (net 8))
 (segment (start 77.47 62.1351) (end 64.77 74.8351) (width 0.25) (layer "B.Cu") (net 8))
 (segment (start 57.0551 80.01) (end 59.5951 77.47) (width 0.25) (layer "B.Cu") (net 8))
 (segment (start 55.88 80.01) (end 57.0551 80.01) (width 0.25) (layer "B.Cu") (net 8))
 (segment (start 57.0904 82.9525) (end 60.325 82.9525) (width 0.25) (layer "F.Cu") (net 7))
 (segment (start 54.5151 80.3772) (end 57.0904 82.9525) (width 0.25) (layer "F.Cu") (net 7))
 (segment (start 53.34 80.01) (end 54.5151 80.01) (width 0.25) (layer "F.Cu") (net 7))
 (segment (start 54.5151 80.01) (end 54.5151 80.3772) (width 0.25) (layer "F.Cu") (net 7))
 (segment (start 102.9649 80.01) (end 102.9649 80.8179) (width 0.25) (layer "F.Cu") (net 5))
 (segment (start 100.8303 82.9525) (end 97.155 82.9525) (width 0.25) (layer "F.Cu") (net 5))
 (segment (start 102.9649 80.8179) (end 100.8303 82.9525) (width 0.25) (layer "F.Cu") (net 5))
 (segment (start 104.14 80.01) (end 102.9649 80.01) (width 0.25) (layer "F.Cu") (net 5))
 (segment (start 60.325 80.8775) (end 60.325 79.105) (width 0.25) (layer "F.Cu") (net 1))
 (segment (start 52.34 71.12) (end 60.325 79.105) (width 0.25) (layer "F.Cu") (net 1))
 (segment (start 43.815 71.12) (end 52.34 71.12) (width 0.25) (layer "F.Cu") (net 1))
 (segment (start 97.155 80.8775) (end 97.155 79.105) (width 0.25) (layer "F.Cu") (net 4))
 (segment (start 98.2288 76.4965) (end 95.6669 73.9346) (width 0.25) (layer "F.Cu") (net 4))
 (segment (start 95.6669 73.9346) (end 90.1156 73.9346) (width 0.25) (layer "F.Cu") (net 4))
 (segment (start 98.2288 78.0312) (end 98.2288 76.4965) (width 0.25) (layer "F.Cu") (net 4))
 (segment (start 90.1156 73.9346) (end 82.221 66.04) (width 0.25) (layer "F.Cu") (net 4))
 (segment (start 82.221 66.04) (end 43.815 66.04) (width 0.25) (layer "F.Cu") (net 4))
 (segment (start 97.155 79.105) (end 98.2288 78.0312) (width 0.25) (layer "F.Cu") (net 4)))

